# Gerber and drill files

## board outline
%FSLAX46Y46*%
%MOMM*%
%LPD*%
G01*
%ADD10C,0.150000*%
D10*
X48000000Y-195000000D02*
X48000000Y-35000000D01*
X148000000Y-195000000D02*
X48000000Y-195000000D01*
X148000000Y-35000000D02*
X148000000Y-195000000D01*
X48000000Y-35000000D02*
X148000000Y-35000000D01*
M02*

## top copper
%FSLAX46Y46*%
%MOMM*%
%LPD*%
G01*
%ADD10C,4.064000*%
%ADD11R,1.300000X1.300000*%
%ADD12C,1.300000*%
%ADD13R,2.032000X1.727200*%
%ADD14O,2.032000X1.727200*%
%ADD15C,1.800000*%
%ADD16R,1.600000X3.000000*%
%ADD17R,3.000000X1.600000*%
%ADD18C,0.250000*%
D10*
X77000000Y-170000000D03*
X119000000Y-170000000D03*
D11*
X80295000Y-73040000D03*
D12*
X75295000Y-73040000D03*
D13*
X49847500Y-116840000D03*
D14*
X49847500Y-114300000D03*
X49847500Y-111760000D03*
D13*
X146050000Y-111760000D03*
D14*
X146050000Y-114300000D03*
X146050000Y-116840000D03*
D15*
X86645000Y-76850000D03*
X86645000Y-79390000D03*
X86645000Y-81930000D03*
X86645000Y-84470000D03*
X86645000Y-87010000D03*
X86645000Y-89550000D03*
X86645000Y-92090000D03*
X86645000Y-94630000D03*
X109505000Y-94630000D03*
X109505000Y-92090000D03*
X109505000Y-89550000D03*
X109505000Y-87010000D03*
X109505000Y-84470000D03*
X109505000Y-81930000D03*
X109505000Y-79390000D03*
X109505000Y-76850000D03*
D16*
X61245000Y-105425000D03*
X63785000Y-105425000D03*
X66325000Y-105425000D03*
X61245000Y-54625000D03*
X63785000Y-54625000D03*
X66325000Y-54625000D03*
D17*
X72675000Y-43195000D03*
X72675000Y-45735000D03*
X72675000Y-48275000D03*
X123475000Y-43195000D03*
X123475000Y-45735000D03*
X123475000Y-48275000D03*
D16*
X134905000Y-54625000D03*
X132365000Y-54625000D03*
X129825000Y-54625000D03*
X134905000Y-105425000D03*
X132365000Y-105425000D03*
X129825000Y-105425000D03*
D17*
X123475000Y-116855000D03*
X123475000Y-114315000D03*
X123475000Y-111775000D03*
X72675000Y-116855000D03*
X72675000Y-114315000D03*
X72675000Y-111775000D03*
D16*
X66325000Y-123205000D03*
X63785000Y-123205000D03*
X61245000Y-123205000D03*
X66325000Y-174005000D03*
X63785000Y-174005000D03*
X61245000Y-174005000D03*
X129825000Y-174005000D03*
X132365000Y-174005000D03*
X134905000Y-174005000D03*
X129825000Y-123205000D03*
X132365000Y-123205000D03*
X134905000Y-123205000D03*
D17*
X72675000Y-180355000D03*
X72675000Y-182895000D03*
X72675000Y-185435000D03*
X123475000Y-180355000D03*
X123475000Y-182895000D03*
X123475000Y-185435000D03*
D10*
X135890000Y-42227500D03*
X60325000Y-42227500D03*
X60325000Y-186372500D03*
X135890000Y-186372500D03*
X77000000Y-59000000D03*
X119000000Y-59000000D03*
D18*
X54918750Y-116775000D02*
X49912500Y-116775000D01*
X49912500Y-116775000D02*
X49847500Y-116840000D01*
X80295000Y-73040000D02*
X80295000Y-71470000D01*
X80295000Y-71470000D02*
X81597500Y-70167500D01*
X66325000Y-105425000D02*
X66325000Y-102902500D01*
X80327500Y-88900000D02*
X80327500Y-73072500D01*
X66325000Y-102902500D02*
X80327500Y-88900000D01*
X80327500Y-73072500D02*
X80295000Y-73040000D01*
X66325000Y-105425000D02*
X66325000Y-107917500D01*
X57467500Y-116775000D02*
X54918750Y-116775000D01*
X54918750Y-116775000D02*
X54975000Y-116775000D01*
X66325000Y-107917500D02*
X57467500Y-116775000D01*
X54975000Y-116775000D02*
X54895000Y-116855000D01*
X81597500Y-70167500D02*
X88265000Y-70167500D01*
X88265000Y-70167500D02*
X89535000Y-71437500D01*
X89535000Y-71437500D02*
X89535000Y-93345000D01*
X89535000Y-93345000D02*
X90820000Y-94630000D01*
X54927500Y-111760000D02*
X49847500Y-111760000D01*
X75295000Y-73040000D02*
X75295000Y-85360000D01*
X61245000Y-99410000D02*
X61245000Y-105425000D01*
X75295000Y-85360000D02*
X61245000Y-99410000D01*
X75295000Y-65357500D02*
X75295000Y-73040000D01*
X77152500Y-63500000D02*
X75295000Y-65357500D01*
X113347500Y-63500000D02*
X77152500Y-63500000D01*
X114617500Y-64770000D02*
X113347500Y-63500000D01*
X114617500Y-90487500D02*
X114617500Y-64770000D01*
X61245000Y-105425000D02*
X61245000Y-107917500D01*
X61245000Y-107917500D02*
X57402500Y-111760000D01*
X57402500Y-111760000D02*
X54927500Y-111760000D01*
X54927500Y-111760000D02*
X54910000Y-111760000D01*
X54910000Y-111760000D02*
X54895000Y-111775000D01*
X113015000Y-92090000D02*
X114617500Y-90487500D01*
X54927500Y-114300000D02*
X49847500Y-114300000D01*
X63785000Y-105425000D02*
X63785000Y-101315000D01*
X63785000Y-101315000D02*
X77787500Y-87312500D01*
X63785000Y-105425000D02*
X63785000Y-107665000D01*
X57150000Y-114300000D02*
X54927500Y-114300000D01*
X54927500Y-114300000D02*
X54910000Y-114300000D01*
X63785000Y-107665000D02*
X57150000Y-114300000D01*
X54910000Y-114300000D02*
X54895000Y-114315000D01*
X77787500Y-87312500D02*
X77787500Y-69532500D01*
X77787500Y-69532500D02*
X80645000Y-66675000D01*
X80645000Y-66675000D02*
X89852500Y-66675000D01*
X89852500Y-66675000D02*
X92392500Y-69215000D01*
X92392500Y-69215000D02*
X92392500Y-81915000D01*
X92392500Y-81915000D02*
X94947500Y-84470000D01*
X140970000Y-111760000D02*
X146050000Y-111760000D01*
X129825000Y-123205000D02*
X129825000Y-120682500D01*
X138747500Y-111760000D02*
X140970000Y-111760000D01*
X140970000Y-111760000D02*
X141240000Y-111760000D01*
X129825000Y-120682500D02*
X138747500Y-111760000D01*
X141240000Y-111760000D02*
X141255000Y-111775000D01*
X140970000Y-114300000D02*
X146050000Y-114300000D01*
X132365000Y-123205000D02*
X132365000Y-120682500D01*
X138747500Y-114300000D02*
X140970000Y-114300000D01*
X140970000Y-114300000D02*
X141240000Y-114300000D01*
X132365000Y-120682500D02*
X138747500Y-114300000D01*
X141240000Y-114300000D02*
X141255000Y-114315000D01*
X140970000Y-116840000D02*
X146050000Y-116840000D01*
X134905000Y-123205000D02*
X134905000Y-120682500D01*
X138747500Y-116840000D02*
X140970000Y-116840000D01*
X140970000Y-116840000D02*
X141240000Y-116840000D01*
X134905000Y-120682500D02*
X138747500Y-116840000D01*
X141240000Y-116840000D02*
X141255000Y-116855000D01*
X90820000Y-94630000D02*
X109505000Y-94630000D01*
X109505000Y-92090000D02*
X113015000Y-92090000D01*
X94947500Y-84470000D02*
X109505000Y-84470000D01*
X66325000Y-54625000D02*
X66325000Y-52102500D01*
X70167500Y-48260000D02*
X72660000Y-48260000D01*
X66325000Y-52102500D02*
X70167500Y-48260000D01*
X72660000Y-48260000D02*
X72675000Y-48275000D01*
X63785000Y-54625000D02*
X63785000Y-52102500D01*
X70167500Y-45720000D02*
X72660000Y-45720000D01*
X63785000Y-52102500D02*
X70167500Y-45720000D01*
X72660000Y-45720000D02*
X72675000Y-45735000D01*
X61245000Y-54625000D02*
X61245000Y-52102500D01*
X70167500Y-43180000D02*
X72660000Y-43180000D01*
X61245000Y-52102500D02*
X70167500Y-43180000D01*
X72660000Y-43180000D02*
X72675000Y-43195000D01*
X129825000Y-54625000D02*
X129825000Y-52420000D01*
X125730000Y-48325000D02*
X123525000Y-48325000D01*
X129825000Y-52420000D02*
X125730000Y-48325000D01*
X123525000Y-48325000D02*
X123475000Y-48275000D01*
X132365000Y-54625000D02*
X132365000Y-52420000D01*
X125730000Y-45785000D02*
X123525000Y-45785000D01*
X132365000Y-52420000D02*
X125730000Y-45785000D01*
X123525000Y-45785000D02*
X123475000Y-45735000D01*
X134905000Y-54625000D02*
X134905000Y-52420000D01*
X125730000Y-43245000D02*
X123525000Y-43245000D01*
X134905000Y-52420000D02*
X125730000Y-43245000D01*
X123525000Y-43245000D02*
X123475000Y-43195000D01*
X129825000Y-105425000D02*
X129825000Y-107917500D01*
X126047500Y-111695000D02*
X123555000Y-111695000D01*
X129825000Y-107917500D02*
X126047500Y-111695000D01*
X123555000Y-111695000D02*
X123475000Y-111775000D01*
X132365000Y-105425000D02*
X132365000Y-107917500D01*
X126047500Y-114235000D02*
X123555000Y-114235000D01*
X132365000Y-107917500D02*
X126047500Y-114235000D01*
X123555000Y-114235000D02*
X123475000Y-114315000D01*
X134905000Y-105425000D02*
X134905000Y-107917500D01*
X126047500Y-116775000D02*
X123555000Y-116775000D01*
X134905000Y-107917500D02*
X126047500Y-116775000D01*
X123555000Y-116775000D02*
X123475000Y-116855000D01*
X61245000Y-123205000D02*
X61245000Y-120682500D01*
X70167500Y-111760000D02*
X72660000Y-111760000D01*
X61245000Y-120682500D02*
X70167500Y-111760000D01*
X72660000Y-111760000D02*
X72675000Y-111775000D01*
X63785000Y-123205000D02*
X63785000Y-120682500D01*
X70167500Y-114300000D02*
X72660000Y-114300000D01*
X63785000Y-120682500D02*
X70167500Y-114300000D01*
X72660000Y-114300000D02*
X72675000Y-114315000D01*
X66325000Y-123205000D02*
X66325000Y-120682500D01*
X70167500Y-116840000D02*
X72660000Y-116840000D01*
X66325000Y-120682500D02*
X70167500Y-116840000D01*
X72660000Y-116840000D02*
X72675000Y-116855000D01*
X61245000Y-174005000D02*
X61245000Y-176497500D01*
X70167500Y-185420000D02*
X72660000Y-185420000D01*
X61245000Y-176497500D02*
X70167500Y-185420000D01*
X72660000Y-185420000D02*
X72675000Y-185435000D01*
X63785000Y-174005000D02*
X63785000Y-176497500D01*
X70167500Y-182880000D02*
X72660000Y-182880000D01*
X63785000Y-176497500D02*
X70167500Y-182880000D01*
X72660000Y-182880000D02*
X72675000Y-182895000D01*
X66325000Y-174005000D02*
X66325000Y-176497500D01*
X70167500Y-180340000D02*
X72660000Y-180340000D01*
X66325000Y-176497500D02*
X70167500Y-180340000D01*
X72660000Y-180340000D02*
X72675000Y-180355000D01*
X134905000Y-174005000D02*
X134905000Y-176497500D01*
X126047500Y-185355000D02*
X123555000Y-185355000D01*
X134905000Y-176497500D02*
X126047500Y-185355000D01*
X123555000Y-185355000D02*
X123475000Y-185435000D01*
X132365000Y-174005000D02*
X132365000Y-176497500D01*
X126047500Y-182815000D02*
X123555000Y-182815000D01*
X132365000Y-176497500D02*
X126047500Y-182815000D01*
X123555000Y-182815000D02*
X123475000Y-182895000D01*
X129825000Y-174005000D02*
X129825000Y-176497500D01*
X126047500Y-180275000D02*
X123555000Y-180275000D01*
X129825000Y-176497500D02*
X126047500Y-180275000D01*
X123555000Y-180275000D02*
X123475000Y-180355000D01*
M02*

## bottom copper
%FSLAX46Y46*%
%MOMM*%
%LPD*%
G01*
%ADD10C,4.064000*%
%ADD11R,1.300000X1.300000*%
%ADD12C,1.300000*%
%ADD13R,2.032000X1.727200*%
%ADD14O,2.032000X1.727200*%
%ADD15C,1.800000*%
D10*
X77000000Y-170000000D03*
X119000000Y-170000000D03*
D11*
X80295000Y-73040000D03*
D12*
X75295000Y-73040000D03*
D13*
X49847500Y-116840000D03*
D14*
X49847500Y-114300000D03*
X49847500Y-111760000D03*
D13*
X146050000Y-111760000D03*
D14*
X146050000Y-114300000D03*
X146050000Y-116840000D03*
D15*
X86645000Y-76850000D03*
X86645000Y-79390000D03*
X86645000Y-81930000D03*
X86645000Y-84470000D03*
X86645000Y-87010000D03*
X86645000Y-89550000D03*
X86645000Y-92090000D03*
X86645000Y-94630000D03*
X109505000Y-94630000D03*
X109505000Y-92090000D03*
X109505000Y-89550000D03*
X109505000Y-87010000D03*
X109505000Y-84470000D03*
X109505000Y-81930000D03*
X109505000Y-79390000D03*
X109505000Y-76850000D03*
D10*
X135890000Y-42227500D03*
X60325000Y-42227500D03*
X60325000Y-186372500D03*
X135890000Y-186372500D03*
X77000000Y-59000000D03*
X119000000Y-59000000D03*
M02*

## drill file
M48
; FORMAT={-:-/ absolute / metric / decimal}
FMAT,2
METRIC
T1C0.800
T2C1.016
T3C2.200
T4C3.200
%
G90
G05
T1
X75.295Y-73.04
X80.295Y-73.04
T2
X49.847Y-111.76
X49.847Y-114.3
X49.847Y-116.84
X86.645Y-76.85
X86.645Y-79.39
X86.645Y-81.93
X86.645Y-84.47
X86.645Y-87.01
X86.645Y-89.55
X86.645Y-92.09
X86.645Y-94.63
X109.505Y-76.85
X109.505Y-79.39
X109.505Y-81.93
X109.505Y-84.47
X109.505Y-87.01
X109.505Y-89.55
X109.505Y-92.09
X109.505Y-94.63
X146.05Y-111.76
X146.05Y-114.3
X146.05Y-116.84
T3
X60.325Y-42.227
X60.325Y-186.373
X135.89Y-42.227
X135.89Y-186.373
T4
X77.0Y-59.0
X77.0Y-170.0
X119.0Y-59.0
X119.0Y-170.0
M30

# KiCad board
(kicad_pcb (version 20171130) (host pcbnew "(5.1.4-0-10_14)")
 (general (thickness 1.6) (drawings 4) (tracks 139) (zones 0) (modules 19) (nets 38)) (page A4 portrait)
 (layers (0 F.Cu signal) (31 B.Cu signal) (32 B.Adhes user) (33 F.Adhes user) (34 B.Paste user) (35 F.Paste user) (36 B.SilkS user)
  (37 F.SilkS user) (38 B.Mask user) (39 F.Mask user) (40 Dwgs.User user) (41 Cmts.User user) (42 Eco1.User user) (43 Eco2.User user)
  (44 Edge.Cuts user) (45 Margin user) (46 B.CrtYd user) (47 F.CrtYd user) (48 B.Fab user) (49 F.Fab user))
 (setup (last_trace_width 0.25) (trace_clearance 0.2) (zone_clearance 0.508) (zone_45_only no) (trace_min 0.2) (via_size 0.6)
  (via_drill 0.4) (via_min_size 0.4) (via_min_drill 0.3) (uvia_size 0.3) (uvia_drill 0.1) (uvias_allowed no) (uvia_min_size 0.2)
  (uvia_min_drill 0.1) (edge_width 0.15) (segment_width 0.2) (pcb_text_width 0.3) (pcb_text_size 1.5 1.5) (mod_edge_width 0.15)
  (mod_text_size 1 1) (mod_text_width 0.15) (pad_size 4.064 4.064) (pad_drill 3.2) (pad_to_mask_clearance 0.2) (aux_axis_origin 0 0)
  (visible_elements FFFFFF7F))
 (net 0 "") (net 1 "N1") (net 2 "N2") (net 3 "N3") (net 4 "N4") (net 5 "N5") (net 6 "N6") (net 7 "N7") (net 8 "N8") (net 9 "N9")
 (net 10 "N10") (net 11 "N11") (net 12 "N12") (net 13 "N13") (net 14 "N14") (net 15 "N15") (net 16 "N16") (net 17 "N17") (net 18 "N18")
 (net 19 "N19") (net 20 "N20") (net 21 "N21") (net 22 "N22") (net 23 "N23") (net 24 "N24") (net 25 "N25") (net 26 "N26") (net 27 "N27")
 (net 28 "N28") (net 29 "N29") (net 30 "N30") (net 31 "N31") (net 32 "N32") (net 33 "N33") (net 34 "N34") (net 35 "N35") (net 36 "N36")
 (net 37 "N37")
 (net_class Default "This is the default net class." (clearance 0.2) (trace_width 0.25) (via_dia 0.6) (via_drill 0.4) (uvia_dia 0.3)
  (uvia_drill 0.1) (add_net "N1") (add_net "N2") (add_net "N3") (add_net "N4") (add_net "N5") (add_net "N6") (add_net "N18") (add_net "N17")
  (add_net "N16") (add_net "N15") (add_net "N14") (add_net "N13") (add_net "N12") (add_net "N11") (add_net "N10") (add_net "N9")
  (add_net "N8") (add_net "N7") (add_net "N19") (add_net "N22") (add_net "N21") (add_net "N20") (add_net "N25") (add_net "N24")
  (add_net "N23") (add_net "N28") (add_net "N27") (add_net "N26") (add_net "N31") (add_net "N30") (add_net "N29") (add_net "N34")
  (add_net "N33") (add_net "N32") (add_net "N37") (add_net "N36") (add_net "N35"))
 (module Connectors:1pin (layer F.Cu) (at 77 170)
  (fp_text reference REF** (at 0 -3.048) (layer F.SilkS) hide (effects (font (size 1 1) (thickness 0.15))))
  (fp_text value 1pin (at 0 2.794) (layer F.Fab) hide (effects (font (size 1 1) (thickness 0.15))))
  (pad 1 thru_hole circle (at 0 0) (size 4.064 4.064) (drill 3.2) (layers F.Cu F.Mask)))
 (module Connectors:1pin (layer F.Cu) (at 119 170)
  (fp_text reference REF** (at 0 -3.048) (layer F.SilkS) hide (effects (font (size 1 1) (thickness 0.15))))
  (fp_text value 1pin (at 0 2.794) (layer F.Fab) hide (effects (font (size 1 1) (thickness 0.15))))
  (pad 1 thru_hole circle (at 0 0) (size 4.064 4.064) (drill 3.2) (layers F.Cu F.Mask)))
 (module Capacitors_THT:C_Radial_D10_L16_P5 (layer F.Cu) (at 80.295 73.04 180)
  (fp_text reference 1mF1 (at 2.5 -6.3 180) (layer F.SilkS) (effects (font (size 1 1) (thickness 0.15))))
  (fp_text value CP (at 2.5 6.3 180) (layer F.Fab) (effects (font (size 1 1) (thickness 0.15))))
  (pad 1 thru_hole rect (at 0 0 180) (size 1.3 1.3) (drill 0.8) (layers F.Cu F.Mask) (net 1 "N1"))
  (pad 2 thru_hole circle (at 5 0 180) (size 1.3 1.3) (drill 0.8) (layers F.Cu F.Mask) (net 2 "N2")))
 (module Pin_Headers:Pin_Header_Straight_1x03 (layer F.Cu) (at 49.8475 116.84 180)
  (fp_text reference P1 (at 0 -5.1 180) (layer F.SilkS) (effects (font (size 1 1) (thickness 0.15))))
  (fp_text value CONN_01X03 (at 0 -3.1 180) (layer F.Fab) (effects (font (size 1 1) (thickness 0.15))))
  (pad 1 thru_hole rect (at 0 0 180) (size 2.032 1.7272) (drill 1.016) (layers F.Cu F.Mask) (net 1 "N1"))
  (pad 2 thru_hole oval (at 0 2.54 180) (size 2.032 1.7272) (drill 1.016) (layers F.Cu F.Mask) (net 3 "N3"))
  (pad 3 thru_hole oval (at 0 5.08 180) (size 2.032 1.7272) (drill 1.016) (layers F.Cu F.Mask) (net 2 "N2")))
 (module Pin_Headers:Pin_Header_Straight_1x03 (layer F.Cu) (at 146.05 111.76)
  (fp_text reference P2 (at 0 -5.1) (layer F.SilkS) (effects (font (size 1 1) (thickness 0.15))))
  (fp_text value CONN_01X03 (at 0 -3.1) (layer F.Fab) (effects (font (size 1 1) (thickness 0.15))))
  (pad 1 thru_hole rect (at 0 0) (size 2.032 1.7272) (drill 1.016) (layers F.Cu F.Mask) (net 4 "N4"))
  (pad 2 thru_hole oval (at 0 2.54) (size 2.032 1.7272) (drill 1.016) (layers F.Cu F.Mask) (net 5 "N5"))
  (pad 3 thru_hole oval (at 0 5.08) (size 2.032 1.7272) (drill 1.016) (layers F.Cu F.Mask) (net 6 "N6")))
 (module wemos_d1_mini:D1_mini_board (layer F.Cu) (at 98.075 87.01)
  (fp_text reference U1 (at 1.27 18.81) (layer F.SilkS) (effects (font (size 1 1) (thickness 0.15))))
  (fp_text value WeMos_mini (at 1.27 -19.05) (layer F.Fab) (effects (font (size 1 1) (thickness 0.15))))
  (pad 8 thru_hole circle (at -11.43 -10.16) (size 1.8 1.8) (drill 1.016) (layers F.Cu F.SilkS F.Mask) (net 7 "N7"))
  (pad 7 thru_hole circle (at -11.43 -7.62) (size 1.8 1.8) (drill 1.016) (layers F.Cu F.SilkS F.Mask) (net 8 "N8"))
  (pad 6 thru_hole circle (at -11.43 -5.08) (size 1.8 1.8) (drill 1.016) (layers F.Cu F.SilkS F.Mask) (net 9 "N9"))
  (pad 5 thru_hole circle (at -11.43 -2.54) (size 1.8 1.8) (drill 1.016) (layers F.Cu F.SilkS F.Mask) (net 3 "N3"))
  (pad 4 thru_hole circle (at -11.43 0) (size 1.8 1.8) (drill 1.016) (layers F.Cu F.SilkS F.Mask) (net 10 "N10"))
  (pad 3 thru_hole circle (at -11.43 2.54) (size 1.8 1.8) (drill 1.016) (layers F.Cu F.SilkS F.Mask) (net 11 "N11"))
  (pad 2 thru_hole circle (at -11.43 5.08) (size 1.8 1.8) (drill 1.016) (layers F.Cu F.SilkS F.Mask) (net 2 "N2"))
  (pad 1 thru_hole circle (at -11.43 7.62) (size 1.8 1.8) (drill 1.016) (layers F.Cu F.SilkS F.Mask) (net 1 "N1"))
  (pad 16 thru_hole circle (at 11.43 7.62) (size 1.8 1.8) (drill 1.016) (layers F.Cu F.SilkS F.Mask) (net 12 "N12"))
  (pad 15 thru_hole circle (at 11.43 5.08) (size 1.8 1.8) (drill 1.016) (layers F.Cu F.SilkS F.Mask) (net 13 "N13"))
  (pad 14 thru_hole circle (at 11.43 2.54) (size 1.8 1.8) (drill 1.016) (layers F.Cu F.SilkS F.Mask) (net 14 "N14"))
  (pad 13 thru_hole circle (at 11.43 0) (size 1.8 1.8) (drill 1.016) (layers F.Cu F.SilkS F.Mask) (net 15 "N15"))
  (pad 12 thru_hole circle (at 11.43 -2.54) (size 1.8 1.8) (drill 1.016) (layers F.Cu F.SilkS F.Mask) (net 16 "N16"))
  (pad 11 thru_hole circle (at 11.43 -5.08) (size 1.8 1.8) (drill 1.016) (layers F.Cu F.SilkS F.Mask) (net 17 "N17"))
  (pad 10 thru_hole circle (at 11.43 -7.62) (size 1.8 1.8) (drill 1.016) (layers F.Cu F.SilkS F.Mask) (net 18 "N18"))
  (pad 9 thru_hole circle (at 11.43 -10.16) (size 1.8 1.8) (drill 1.016) (layers F.Cu F.SilkS F.Mask) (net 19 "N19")))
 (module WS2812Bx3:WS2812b (layer F.Cu) (at 63.785 80.025 90)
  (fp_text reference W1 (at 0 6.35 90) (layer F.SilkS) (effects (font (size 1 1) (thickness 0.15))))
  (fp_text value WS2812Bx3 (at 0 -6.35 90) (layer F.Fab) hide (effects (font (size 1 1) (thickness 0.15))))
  (pad 1 smd rect (at -25.4 -2.54 90) (size 3 1.6) (layers F.Cu F.Paste F.Mask) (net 2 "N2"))
  (pad 2 smd rect (at -25.4 0 90) (size 3 1.6) (layers F.Cu F.Paste F.Mask) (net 3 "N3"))
  (pad 3 smd rect (at -25.4 2.54 90) (size 3 1.6) (layers F.Cu F.Paste F.Mask) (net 1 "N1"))
  (pad 6 smd rect (at 25.4 -2.54 90) (size 3 1.6) (layers F.Cu F.Paste F.Mask) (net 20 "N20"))
  (pad 5 smd rect (at 25.4 0 90) (size 3 1.6) (layers F.Cu F.Paste F.Mask) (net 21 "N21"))
  (pad 4 smd rect (at 25.4 2.54 90) (size 3 1.6) (layers F.Cu F.Paste F.Mask) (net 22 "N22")))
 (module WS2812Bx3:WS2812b (layer F.Cu) (at 98.075 45.735)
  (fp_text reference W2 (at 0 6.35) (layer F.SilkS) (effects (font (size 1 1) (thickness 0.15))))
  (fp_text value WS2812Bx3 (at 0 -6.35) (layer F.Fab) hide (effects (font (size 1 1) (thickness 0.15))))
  (pad 1 smd rect (at -25.4 -2.54) (size 3 1.6) (layers F.Cu F.Paste F.Mask) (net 20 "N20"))
  (pad 2 smd rect (at -25.4 0) (size 3 1.6) (layers F.Cu F.Paste F.Mask) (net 21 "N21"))
  (pad 3 smd rect (at -25.4 2.54) (size 3 1.6) (layers F.Cu F.Paste F.Mask) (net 22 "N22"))
  (pad 6 smd rect (at 25.4 -2.54) (size 3 1.6) (layers F.Cu F.Paste F.Mask) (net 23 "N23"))
  (pad 5 smd rect (at 25.4 0) (size 3 1.6) (layers F.Cu F.Paste F.Mask) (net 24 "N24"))
  (pad 4 smd rect (at 25.4 2.54) (size 3 1.6) (layers F.Cu F.Paste F.Mask) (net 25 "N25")))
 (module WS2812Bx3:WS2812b (layer F.Cu) (at 132.365 80.025 270)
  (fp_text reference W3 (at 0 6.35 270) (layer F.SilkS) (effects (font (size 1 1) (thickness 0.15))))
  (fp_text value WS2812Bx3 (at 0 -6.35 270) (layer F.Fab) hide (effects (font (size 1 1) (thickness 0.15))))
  (pad 1 smd rect (at -25.4 -2.54 270) (size 3 1.6) (layers F.Cu F.Paste F.Mask) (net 23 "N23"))
  (pad 2 smd rect (at -25.4 0 270) (size 3 1.6) (layers F.Cu F.Paste F.Mask) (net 24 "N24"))
  (pad 3 smd rect (at -25.4 2.54 270) (size 3 1.6) (layers F.Cu F.Paste F.Mask) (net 25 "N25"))
  (pad 6 smd rect (at 25.4 -2.54 270) (size 3 1.6) (layers F.Cu F.Paste F.Mask) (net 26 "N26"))
  (pad 5 smd rect (at 25.4 0 270) (size 3 1.6) (layers F.Cu F.Paste F.Mask) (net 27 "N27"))
  (pad 4 smd rect (at 25.4 2.54 270) (size 3 1.6) (layers F.Cu F.Paste F.Mask) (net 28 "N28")))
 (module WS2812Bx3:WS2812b (layer F.Cu) (at 98.075 114.315 180)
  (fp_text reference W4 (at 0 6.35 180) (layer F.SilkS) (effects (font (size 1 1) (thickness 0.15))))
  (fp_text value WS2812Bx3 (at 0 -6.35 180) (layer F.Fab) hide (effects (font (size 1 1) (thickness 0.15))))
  (pad 1 smd rect (at -25.4 -2.54 180) (size 3 1.6) (layers F.Cu F.Paste F.Mask) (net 26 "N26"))
  (pad 2 smd rect (at -25.4 0 180) (size 3 1.6) (layers F.Cu F.Paste F.Mask) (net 27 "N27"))
  (pad 3 smd rect (at -25.4 2.54 180) (size 3 1.6) (layers F.Cu F.Paste F.Mask) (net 28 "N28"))
  (pad 6 smd rect (at 25.4 -2.54 180) (size 3 1.6) (layers F.Cu F.Paste F.Mask) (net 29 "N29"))
  (pad 5 smd rect (at 25.4 0 180) (size 3 1.6) (layers F.Cu F.Paste F.Mask) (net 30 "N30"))
  (pad 4 smd rect (at 25.4 2.54 180) (size 3 1.6) (layers F.Cu F.Paste F.Mask) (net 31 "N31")))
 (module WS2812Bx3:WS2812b (layer F.Cu) (at 63.785 148.605 270)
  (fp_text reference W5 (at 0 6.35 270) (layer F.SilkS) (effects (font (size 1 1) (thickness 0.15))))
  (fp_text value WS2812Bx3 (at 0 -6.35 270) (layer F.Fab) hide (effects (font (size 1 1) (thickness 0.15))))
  (pad 1 smd rect (at -25.4 -2.54 270) (size 3 1.6) (layers F.Cu F.Paste F.Mask) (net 29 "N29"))
  (pad 2 smd rect (at -25.4 0 270) (size 3 1.6) (layers F.Cu F.Paste F.Mask) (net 30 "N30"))
  (pad 3 smd rect (at -25.4 2.54 270) (size 3 1.6) (layers F.Cu F.Paste F.Mask) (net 31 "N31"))
  (pad 6 smd rect (at 25.4 -2.54 270) (size 3 1.6) (layers F.Cu F.Paste F.Mask) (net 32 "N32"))
  (pad 5 smd rect (at 25.4 0 270) (size 3 1.6) (layers F.Cu F.Paste F.Mask) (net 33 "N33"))
  (pad 4 smd rect (at 25.4 2.54 270) (size 3 1.6) (layers F.Cu F.Paste F.Mask) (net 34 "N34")))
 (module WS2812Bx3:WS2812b (layer F.Cu) (at 132.365 148.605 90)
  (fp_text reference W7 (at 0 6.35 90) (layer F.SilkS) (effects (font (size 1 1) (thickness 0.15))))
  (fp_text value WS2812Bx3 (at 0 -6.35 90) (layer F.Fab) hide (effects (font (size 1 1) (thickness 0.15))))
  (pad 1 smd rect (at -25.4 -2.54 90) (size 3 1.6) (layers F.Cu F.Paste F.Mask) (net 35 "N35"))
  (pad 2 smd rect (at -25.4 0 90) (size 3 1.6) (layers F.Cu F.Paste F.Mask) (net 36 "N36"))
  (pad 3 smd rect (at -25.4 2.54 90) (size 3 1.6) (layers F.Cu F.Paste F.Mask) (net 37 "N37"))
  (pad 6 smd rect (at 25.4 -2.54 90) (size 3 1.6) (layers F.Cu F.Paste F.Mask) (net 4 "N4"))
  (pad 5 smd rect (at 25.4 0 90) (size 3 1.6) (layers F.Cu F.Paste F.Mask) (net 5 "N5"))
  (pad 4 smd rect (at 25.4 2.54 90) (size 3 1.6) (layers F.Cu F.Paste F.Mask) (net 6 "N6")))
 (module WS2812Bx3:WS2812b (layer F.Cu) (at 98.075 182.895)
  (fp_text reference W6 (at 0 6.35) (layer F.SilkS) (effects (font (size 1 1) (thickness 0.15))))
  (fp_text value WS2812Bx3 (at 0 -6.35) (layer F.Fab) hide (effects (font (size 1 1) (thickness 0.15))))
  (pad 1 smd rect (at -25.4 -2.54) (size 3 1.6) (layers F.Cu F.Paste F.Mask) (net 32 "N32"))
  (pad 2 smd rect (at -25.4 0) (size 3 1.6) (layers F.Cu F.Paste F.Mask) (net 33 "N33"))
  (pad 3 smd rect (at -25.4 2.54) (size 3 1.6) (layers F.Cu F.Paste F.Mask) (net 34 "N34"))
  (pad 6 smd rect (at 25.4 -2.54) (size 3 1.6) (layers F.Cu F.Paste F.Mask) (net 35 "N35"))
  (pad 5 smd rect (at 25.4 0) (size 3 1.6) (layers F.Cu F.Paste F.Mask) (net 36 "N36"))
  (pad 4 smd rect (at 25.4 2.54) (size 3 1.6) (layers F.Cu F.Paste F.Mask) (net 37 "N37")))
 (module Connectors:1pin (layer F.Cu) (at 135.89 42.2275)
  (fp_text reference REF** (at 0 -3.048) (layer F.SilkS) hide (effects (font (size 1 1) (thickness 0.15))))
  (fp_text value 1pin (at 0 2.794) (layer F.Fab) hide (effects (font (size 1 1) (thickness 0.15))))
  (pad 1 thru_hole circle (at 0 0) (size 4.064 4.064) (drill 2.2) (layers F.Cu F.Mask)))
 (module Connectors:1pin (layer F.Cu) (at 60.325 42.2275)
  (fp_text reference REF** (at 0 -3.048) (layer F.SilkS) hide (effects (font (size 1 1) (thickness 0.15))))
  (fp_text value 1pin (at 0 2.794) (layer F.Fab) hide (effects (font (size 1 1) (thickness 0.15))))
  (pad 1 thru_hole circle (at 0 0) (size 4.064 4.064) (drill 2.2) (layers F.Cu F.Mask)))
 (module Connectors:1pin (layer F.Cu) (at 60.325 186.3725)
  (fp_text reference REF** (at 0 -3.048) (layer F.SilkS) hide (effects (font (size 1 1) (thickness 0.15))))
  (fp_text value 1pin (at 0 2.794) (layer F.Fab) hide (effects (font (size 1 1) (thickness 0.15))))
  (pad 1 thru_hole circle (at 0 0) (size 4.064 4.064) (drill 2.2) (layers F.Cu F.Mask)))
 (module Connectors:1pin (layer F.Cu) (at 135.89 186.3725)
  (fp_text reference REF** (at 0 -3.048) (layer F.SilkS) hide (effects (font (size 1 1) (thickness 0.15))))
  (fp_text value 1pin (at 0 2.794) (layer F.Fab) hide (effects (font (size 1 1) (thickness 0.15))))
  (pad 1 thru_hole circle (at 0 0) (size 4.064 4.064) (drill 2.2) (layers F.Cu F.Mask)))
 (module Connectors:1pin (layer F.Cu) (at 77 59)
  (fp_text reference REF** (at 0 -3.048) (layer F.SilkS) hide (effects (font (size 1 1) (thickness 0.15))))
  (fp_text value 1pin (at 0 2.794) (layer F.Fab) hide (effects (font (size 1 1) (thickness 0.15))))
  (pad 1 thru_hole circle (at 0 0) (size 4.064 4.064) (drill 3.2) (layers F.Cu F.Mask)))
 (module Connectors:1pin (layer F.Cu) (at 119 59)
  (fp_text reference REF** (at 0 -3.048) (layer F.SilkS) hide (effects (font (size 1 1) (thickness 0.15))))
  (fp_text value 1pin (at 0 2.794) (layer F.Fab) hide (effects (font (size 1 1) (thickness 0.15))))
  (pad 1 thru_hole circle (at 0 0) (size 4.064 4.064) (drill 3.2) (layers F.Cu F.Mask)))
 (gr_line (start 48 195) (end 48 35) (angle 90) (layer Edge.Cuts) (width 0.15))
 (gr_line (start 148 195) (end 48 195) (angle 90) (layer Edge.Cuts) (width 0.15))
 (gr_line (start 148 35) (end 148 195) (angle 90) (layer Edge.Cuts) (width 0.15))
 (gr_line (start 48 35) (end 148 35) (angle 90) (layer Edge.Cuts) (width 0.15))
 (segment (start 54.91875 116.775) (end 49.9125 116.775) (width 0.25) (layer F.Cu) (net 1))
 (segment (start 49.9125 116.775) (end 49.8475 116.84) (width 0.25) (layer F.Cu) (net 1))
 (segment (start 80.295 73.04) (end 80.295 71.47) (width 0.25) (layer F.Cu) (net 1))
 (segment (start 80.295 71.47) (end 81.5975 70.1675) (width 0.25) (layer F.Cu) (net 1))
 (segment (start 66.325 105.425) (end 66.325 102.9025) (width 0.25) (layer F.Cu) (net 1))
 (segment (start 80.3275 88.9) (end 80.3275 73.0725) (width 0.25) (layer F.Cu) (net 1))
 (segment (start 66.325 102.9025) (end 80.3275 88.9) (width 0.25) (layer F.Cu) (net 1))
 (segment (start 80.3275 73.0725) (end 80.295 73.04) (width 0.25) (layer F.Cu) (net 1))
 (segment (start 66.325 105.425) (end 66.325 107.9175) (width 0.25) (layer F.Cu) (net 1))
 (segment (start 57.4675 116.775) (end 54.91875 116.775) (width 0.25) (layer F.Cu) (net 1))
 (segment (start 54.91875 116.775) (end 54.975 116.775) (width 0.25) (layer F.Cu) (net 1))
 (segment (start 66.325 107.9175) (end 57.4675 116.775) (width 0.25) (layer F.Cu) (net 1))
 (segment (start 54.975 116.775) (end 54.895 116.855) (width 0.25) (layer F.Cu) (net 1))
 (segment (start 81.5975 70.1675) (end 88.265 70.1675) (width 0.25) (layer F.Cu) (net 1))
 (segment (start 88.265 70.1675) (end 89.535 71.4375) (width 0.25) (layer F.Cu) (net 1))
 (segment (start 89.535 71.4375) (end 89.535 93.345) (width 0.25) (layer F.Cu) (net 1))
 (segment (start 89.535 93.345) (end 90.82 94.63) (width 0.25) (layer F.Cu) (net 1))
 (segment (start 54.9275 111.76) (end 49.8475 111.76) (width 0.25) (layer F.Cu) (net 2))
 (segment (start 75.295 73.04) (end 75.295 85.36) (width 0.25) (layer F.Cu) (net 2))
 (segment (start 61.245 99.41) (end 61.245 105.425) (width 0.25) (layer F.Cu) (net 2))
 (segment (start 75.295 85.36) (end 61.245 99.41) (width 0.25) (layer F.Cu) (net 2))
 (segment (start 75.295 65.3575) (end 75.295 73.04) (width 0.25) (layer F.Cu) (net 2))
 (segment (start 77.1525 63.5) (end 75.295 65.3575) (width 0.25) (layer F.Cu) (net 2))
 (segment (start 113.3475 63.5) (end 77.1525 63.5) (width 0.25) (layer F.Cu) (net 2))
 (segment (start 114.6175 64.77) (end 113.3475 63.5) (width 0.25) (layer F.Cu) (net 2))
 (segment (start 114.6175 90.4875) (end 114.6175 64.77) (width 0.25) (layer F.Cu) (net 2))
 (segment (start 61.245 105.425) (end 61.245 107.9175) (width 0.25) (layer F.Cu) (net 2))
 (segment (start 61.245 107.9175) (end 57.4025 111.76) (width 0.25) (layer F.Cu) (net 2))
 (segment (start 57.4025 111.76) (end 54.9275 111.76) (width 0.25) (layer F.Cu) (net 2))
 (segment (start 54.9275 111.76) (end 54.91 111.76) (width 0.25) (layer F.Cu) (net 2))
 (segment (start 54.91 111.76) (end 54.895 111.775) (width 0.25) (layer F.Cu) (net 2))
 (segment (start 113.015 92.09) (end 114.6175 90.4875) (width 0.25) (layer F.Cu) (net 2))
 (segment (start 54.9275 114.3) (end 49.8475 114.3) (width 0.25) (layer F.Cu) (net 3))
 (segment (start 63.785 105.425) (end 63.785 101.315) (width 0.25) (layer F.Cu) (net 3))
 (segment (start 63.785 101.315) (end 77.7875 87.3125) (width 0.25) (layer F.Cu) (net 3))
 (segment (start 63.785 105.425) (end 63.785 107.665) (width 0.25) (layer F.Cu) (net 3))
 (segment (start 57.15 114.3) (end 54.9275 114.3) (width 0.25) (layer F.Cu) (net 3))
 (segment (start 54.9275 114.3) (end 54.91 114.3) (width 0.25) (layer F.Cu) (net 3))
 (segment (start 63.785 107.665) (end 57.15 114.3) (width 0.25) (layer F.Cu) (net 3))
 (segment (start 54.91 114.3) (end 54.895 114.315) (width 0.25) (layer F.Cu) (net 3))
 (segment (start 77.7875 87.3125) (end 77.7875 69.5325) (width 0.25) (layer F.Cu) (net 3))
 (segment (start 77.7875 69.5325) (end 80.645 66.675) (width 0.25) (layer F.Cu) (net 3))
 (segment (start 80.645 66.675) (end 89.8525 66.675) (width 0.25) (layer F.Cu) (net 3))
 (segment (start 89.8525 66.675) (end 92.3925 69.215) (width 0.25) (layer F.Cu) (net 3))
 (segment (start 92.3925 69.215) (end 92.3925 81.915) (width 0.25) (layer F.Cu) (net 3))
 (segment (start 92.3925 81.915) (end 94.9475 84.47) (width 0.25) (layer F.Cu) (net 3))
 (segment (start 140.97 111.76) (end 146.05 111.76) (width 0.25) (layer F.Cu) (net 4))
 (segment (start 129.825 123.205) (end 129.825 120.6825) (width 0.25) (layer F.Cu) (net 4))
 (segment (start 138.7475 111.76) (end 140.97 111.76) (width 0.25) (layer F.Cu) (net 4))
 (segment (start 140.97 111.76) (end 141.24 111.76) (width 0.25) (layer F.Cu) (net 4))
 (segment (start 129.825 120.6825) (end 138.7475 111.76) (width 0.25) (layer F.Cu) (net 4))
 (segment (start 141.24 111.76) (end 141.255 111.775) (width 0.25) (layer F.Cu) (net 4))
 (segment (start 140.97 114.3) (end 146.05 114.3) (width 0.25) (layer F.Cu) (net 5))
 (segment (start 132.365 123.205) (end 132.365 120.6825) (width 0.25) (layer F.Cu) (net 5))
 (segment (start 138.7475 114.3) (end 140.97 114.3) (width 0.25) (layer F.Cu) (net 5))
 (segment (start 140.97 114.3) (end 141.24 114.3) (width 0.25) (layer F.Cu) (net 5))
 (segment (start 132.365 120.6825) (end 138.7475 114.3) (width 0.25) (layer F.Cu) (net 5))
 (segment (start 141.24 114.3) (end 141.255 114.315) (width 0.25) (layer F.Cu) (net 5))
 (segment (start 140.97 116.84) (end 146.05 116.84) (width 0.25) (layer F.Cu) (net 6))
 (segment (start 134.905 123.205) (end 134.905 120.6825) (width 0.25) (layer F.Cu) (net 6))
 (segment (start 138.7475 116.84) (end 140.97 116.84) (width 0.25) (layer F.Cu) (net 6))
 (segment (start 140.97 116.84) (end 141.24 116.84) (width 0.25) (layer F.Cu) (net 6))
 (segment (start 134.905 120.6825) (end 138.7475 116.84) (width 0.25) (layer F.Cu) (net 6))
 (segment (start 141.24 116.84) (end 141.255 116.855) (width 0.25) (layer F.Cu) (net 6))
 (segment (start 90.82 94.63) (end 109.505 94.63) (width 0.25) (layer F.Cu) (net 12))
 (segment (start 109.505 92.09) (end 113.015 92.09) (width 0.25) (layer F.Cu) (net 13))
 (segment (start 94.9475 84.47) (end 109.505 84.47) (width 0.25) (layer F.Cu) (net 16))
 (segment (start 66.325 54.625) (end 66.325 52.1025) (width 0.25) (layer F.Cu) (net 22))
 (segment (start 70.1675 48.26) (end 72.66 48.26) (width 0.25) (layer F.Cu) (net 22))
 (segment (start 66.325 52.1025) (end 70.1675 48.26) (width 0.25) (layer F.Cu) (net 22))
 (segment (start 72.66 48.26) (end 72.675 48.275) (width 0.25) (layer F.Cu) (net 22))
 (segment (start 63.785 54.625) (end 63.785 52.1025) (width 0.25) (layer F.Cu) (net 21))
 (segment (start 70.1675 45.72) (end 72.66 45.72) (width 0.25) (layer F.Cu) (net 21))
 (segment (start 63.785 52.1025) (end 70.1675 45.72) (width 0.25) (layer F.Cu) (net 21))
 (segment (start 72.66 45.72) (end 72.675 45.735) (width 0.25) (layer F.Cu) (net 21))
 (segment (start 61.245 54.625) (end 61.245 52.1025) (width 0.25) (layer F.Cu) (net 20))
 (segment (start 70.1675 43.18) (end 72.66 43.18) (width 0.25) (layer F.Cu) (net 20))
 (segment (start 61.245 52.1025) (end 70.1675 43.18) (width 0.25) (layer F.Cu) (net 20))
 (segment (start 72.66 43.18) (end 72.675 43.195) (width 0.25) (layer F.Cu) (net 20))
 (segment (start 129.825 54.625) (end 129.825 52.42) (width 0.25) (layer F.Cu) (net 25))
 (segment (start 125.73 48.325) (end 123.525 48.325) (width 0.25) (layer F.Cu) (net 25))
 (segment (start 129.825 52.42) (end 125.73 48.325) (width 0.25) (layer F.Cu) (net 25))
 (segment (start 123.525 48.325) (end 123.475 48.275) (width 0.25) (layer F.Cu) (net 25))
 (segment (start 132.365 54.625) (end 132.365 52.42) (width 0.25) (layer F.Cu) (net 24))
 (segment (start 125.73 45.785) (end 123.525 45.785) (width 0.25) (layer F.Cu) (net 24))
 (segment (start 132.365 52.42) (end 125.73 45.785) (width 0.25) (layer F.Cu) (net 24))
 (segment (start 123.525 45.785) (end 123.475 45.735) (width 0.25) (layer F.Cu) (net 24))
 (segment (start 134.905 54.625) (end 134.905 52.42) (width 0.25) (layer F.Cu) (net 23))
 (segment (start 125.73 43.245) (end 123.525 43.245) (width 0.25) (layer F.Cu) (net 23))
 (segment (start 134.905 52.42) (end 125.73 43.245) (width 0.25) (layer F.Cu) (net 23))
 (segment (start 123.525 43.245) (end 123.475 43.195) (width 0.25) (layer F.Cu) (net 23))
 (segment (start 129.825 105.425) (end 129.825 107.9175) (width 0.25) (layer F.Cu) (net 28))
 (segment (start 126.0475 111.695) (end 123.555 111.695) (width 0.25) (layer F.Cu) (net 28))
 (segment (start 129.825 107.9175) (end 126.0475 111.695) (width 0.25) (layer F.Cu) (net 28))
 (segment (start 123.555 111.695) (end 123.475 111.775) (width 0.25) (layer F.Cu) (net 28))
 (segment (start 132.365 105.425) (end 132.365 107.9175) (width 0.25) (layer F.Cu) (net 27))
 (segment (start 126.0475 114.235) (end 123.555 114.235) (width 0.25) (layer F.Cu) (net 27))
 (segment (start 132.365 107.9175) (end 126.0475 114.235) (width 0.25) (layer F.Cu) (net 27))
 (segment (start 123.555 114.235) (end 123.475 114.315) (width 0.25) (layer F.Cu) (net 27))
 (segment (start 134.905 105.425) (end 134.905 107.9175) (width 0.25) (layer F.Cu) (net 26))
 (segment (start 126.0475 116.775) (end 123.555 116.775) (width 0.25) (layer F.Cu) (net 26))
 (segment (start 134.905 107.9175) (end 126.0475 116.775) (width 0.25) (layer F.Cu) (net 26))
 (segment (start 123.555 116.775) (end 123.475 116.855) (width 0.25) (layer F.Cu) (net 26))
 (segment (start 61.245 123.205) (end 61.245 120.6825) (width 0.25) (layer F.Cu) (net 31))
 (segment (start 70.1675 111.76) (end 72.66 111.76) (width 0.25) (layer F.Cu) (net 31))
 (segment (start 61.245 120.6825) (end 70.1675 111.76) (width 0.25) (layer F.Cu) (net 31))
 (segment (start 72.66 111.76) (end 72.675 111.775) (width 0.25) (layer F.Cu) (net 31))
 (segment (start 63.785 123.205) (end 63.785 120.6825) (width 0.25) (layer F.Cu) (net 30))
 (segment (start 70.1675 114.3) (end 72.66 114.3) (width 0.25) (layer F.Cu) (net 30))
 (segment (start 63.785 120.6825) (end 70.1675 114.3) (width 0.25) (layer F.Cu) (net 30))
 (segment (start 72.66 114.3) (end 72.675 114.315) (width 0.25) (layer F.Cu) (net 30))
 (segment (start 66.325 123.205) (end 66.325 120.6825) (width 0.25) (layer F.Cu) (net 29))
 (segment (start 70.1675 116.84) (end 72.66 116.84) (width 0.25) (layer F.Cu) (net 29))
 (segment (start 66.325 120.6825) (end 70.1675 116.84) (width 0.25) (layer F.Cu) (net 29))
 (segment (start 72.66 116.84) (end 72.675 116.855) (width 0.25) (layer F.Cu) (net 29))
 (segment (start 61.245 174.005) (end 61.245 176.4975) (width 0.25) (layer F.Cu) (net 34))
 (segment (start 70.1675 185.42) (end 72.66 185.42) (width 0.25) (layer F.Cu) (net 34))
 (segment (start 61.245 176.4975) (end 70.1675 185.42) (width 0.25) (layer F.Cu) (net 34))
 (segment (start 72.66 185.42) (end 72.675 185.435) (width 0.25) (layer F.Cu) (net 34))
 (segment (start 63.785 174.005) (end 63.785 176.4975) (width 0.25) (layer F.Cu) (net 33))
 (segment (start 70.1675 182.88) (end 72.66 182.88) (width 0.25) (layer F.Cu) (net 33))
 (segment (start 63.785 176.4975) (end 70.1675 182.88) (width 0.25) (layer F.Cu) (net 33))
 (segment (start 72.66 182.88) (end 72.675 182.895) (width 0.25) (layer F.Cu) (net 33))
 (segment (start 66.325 174.005) (end 66.325 176.4975) (width 0.25) (layer F.Cu) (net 32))
 (segment (start 70.1675 180.34) (end 72.66 180.34) (width 0.25) (layer F.Cu) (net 32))
 (segment (start 66.325 176.4975) (end 70.1675 180.34) (width 0.25) (layer F.Cu) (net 32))
 (segment (start 72.66 180.34) (end 72.675 180.355) (width 0.25) (layer F.Cu) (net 32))
 (segment (start 134.905 174.005) (end 134.905 176.4975) (width 0.25) (layer F.Cu) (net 37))
 (segment (start 126.0475 185.355) (end 123.555 185.355) (width 0.25) (layer F.Cu) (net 37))
 (segment (start 134.905 176.4975) (end 126.0475 185.355) (width 0.25) (layer F.Cu) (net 37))
 (segment (start 123.555 185.355) (end 123.475 185.435) (width 0.25) (layer F.Cu) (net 37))
 (segment (start 132.365 174.005) (end 132.365 176.4975) (width 0.25) (layer F.Cu) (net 36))
 (segment (start 126.0475 182.815) (end 123.555 182.815) (width 0.25) (layer F.Cu) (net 36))
 (segment (start 132.365 176.4975) (end 126.0475 182.815) (width 0.25) (layer F.Cu) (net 36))
 (segment (start 123.555 182.815) (end 123.475 182.895) (width 0.25) (layer F.Cu) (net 36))
 (segment (start 129.825 174.005) (end 129.825 176.4975) (width 0.25) (layer F.Cu) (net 35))
 (segment (start 126.0475 180.275) (end 123.555 180.275) (width 0.25) (layer F.Cu) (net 35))
 (segment (start 129.825 176.4975) (end 126.0475 180.275) (width 0.25) (layer F.Cu) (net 35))
 (segment (start 123.555 180.275) (end 123.475 180.355) (width 0.25) (layer F.Cu) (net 35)))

